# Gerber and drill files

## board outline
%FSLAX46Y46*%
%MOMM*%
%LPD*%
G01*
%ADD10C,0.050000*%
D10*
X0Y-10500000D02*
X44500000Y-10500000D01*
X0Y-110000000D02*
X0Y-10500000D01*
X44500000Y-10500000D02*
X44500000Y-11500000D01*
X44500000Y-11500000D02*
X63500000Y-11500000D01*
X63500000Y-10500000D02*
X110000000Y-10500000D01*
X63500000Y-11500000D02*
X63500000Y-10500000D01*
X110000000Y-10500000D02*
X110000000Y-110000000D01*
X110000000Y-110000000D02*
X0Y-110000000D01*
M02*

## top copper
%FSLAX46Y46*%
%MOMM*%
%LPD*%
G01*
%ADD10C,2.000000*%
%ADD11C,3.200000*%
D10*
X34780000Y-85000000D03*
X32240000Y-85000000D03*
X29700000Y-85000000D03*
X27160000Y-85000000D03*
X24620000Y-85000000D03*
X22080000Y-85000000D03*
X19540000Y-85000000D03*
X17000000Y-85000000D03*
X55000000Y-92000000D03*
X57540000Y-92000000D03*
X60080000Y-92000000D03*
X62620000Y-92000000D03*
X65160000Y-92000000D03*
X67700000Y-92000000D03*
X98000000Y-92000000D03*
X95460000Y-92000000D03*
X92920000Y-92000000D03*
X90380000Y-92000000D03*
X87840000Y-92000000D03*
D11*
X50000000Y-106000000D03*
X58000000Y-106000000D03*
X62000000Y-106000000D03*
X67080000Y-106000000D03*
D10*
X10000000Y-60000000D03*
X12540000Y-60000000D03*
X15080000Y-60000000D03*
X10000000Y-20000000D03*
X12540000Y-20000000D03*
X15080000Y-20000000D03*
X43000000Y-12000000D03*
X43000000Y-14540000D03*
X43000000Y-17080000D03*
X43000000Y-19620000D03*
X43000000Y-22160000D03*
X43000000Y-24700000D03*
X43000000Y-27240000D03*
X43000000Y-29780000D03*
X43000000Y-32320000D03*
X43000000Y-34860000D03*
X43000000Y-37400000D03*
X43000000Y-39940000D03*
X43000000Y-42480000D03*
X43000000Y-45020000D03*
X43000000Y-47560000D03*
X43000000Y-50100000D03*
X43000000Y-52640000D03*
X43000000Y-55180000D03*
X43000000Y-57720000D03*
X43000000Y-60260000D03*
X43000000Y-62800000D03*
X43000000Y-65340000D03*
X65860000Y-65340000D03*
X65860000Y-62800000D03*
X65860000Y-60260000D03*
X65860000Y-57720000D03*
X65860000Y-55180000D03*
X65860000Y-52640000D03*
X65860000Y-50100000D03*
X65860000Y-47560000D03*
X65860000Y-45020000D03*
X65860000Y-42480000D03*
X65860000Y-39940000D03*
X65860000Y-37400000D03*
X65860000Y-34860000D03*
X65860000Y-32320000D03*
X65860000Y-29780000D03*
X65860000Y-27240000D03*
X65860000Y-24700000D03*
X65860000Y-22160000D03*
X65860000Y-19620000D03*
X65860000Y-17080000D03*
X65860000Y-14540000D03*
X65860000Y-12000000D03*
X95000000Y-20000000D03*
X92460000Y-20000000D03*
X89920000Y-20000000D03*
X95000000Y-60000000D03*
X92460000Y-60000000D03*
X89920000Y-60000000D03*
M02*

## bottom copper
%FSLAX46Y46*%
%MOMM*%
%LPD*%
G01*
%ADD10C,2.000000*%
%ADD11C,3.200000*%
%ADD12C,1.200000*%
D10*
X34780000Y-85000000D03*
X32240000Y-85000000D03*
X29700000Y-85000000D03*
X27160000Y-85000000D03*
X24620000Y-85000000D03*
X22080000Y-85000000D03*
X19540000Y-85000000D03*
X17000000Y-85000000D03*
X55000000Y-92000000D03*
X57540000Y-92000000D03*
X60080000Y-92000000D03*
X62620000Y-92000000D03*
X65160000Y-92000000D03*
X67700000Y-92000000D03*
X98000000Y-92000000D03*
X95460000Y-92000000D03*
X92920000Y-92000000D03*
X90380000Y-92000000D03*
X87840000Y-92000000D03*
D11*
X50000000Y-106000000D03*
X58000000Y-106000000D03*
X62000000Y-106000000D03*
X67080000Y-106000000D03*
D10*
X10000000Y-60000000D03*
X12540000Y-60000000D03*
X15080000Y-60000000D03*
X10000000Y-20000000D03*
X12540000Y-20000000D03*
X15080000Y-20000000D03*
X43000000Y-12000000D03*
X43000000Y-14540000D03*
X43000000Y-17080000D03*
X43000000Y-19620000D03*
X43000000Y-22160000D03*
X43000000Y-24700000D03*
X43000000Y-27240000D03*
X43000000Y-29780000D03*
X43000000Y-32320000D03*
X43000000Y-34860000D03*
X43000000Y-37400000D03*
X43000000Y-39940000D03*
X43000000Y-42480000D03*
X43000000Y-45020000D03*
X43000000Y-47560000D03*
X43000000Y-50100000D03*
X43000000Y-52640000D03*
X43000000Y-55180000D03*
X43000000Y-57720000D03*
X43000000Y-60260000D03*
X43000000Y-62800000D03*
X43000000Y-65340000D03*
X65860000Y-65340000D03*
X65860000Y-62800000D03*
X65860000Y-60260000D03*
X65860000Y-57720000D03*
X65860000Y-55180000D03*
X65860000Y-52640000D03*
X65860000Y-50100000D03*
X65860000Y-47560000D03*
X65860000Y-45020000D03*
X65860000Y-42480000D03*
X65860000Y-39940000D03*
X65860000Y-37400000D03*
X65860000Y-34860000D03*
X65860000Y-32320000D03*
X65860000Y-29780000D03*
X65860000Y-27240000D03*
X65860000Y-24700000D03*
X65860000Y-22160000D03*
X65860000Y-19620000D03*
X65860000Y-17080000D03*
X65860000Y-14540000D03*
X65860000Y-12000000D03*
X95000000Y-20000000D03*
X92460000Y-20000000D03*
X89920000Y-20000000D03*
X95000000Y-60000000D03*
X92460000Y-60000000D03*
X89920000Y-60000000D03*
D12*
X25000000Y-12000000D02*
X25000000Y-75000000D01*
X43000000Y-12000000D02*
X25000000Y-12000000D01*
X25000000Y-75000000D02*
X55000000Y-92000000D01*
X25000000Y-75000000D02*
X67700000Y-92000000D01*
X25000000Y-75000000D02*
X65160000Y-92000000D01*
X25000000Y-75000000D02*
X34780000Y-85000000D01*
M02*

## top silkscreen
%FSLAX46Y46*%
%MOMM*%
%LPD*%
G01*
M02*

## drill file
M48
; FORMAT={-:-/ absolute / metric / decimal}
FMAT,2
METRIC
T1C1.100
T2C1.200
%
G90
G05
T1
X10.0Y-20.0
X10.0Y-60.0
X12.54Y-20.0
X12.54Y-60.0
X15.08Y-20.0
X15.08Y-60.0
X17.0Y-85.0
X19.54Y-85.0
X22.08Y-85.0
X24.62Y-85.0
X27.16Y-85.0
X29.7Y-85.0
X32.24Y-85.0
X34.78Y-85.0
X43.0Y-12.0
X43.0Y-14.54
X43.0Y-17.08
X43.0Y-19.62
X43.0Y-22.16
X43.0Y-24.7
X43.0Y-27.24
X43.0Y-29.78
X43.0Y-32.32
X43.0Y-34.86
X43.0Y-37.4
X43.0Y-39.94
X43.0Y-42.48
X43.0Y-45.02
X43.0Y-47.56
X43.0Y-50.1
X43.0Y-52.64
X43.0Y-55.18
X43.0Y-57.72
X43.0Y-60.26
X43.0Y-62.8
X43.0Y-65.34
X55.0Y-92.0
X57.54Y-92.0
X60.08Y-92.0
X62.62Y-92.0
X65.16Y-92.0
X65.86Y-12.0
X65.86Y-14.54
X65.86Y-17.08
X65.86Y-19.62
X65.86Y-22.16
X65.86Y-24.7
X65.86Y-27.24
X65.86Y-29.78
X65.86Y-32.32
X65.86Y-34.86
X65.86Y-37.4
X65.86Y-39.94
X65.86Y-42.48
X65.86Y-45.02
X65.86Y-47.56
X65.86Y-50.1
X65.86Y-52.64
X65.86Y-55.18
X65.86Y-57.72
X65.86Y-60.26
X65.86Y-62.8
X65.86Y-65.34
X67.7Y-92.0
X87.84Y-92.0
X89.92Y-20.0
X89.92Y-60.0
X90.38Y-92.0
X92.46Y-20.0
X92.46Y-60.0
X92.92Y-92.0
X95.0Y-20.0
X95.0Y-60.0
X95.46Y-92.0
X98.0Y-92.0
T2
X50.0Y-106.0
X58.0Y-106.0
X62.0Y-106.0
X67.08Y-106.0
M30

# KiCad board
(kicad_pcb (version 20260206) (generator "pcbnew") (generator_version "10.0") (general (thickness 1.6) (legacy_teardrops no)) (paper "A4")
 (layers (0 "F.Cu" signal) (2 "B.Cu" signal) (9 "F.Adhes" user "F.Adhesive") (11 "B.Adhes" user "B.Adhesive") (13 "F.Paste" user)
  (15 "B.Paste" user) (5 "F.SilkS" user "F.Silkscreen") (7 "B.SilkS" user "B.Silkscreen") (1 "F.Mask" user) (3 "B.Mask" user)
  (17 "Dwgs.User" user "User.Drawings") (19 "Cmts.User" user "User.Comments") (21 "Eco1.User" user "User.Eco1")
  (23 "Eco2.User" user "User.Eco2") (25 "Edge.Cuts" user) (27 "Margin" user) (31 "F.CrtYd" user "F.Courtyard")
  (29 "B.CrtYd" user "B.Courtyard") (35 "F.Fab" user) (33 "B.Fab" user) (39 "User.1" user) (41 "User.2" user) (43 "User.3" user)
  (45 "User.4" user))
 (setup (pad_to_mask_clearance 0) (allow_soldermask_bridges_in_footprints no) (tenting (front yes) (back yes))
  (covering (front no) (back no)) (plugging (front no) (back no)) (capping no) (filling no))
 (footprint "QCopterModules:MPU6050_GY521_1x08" (layer "F.Cu") (at 34.78 85 -90)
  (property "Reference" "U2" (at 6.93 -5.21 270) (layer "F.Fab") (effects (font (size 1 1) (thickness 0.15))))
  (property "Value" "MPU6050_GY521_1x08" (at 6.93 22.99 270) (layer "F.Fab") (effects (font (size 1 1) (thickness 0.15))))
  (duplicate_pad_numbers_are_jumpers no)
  (pad "1" thru_hole circle (at 0 0 270) (size 2 2) (drill 1.1) (layers "*.Cu" "*.Mask") (remove_unused_layers no) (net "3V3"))
  (pad "2" thru_hole circle (at 0 2.54 270) (size 2 2) (drill 1.1) (layers "*.Cu" "*.Mask") (remove_unused_layers no) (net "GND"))
  (pad "3" thru_hole circle (at 0 5.08 270) (size 2 2) (drill 1.1) (layers "*.Cu" "*.Mask") (remove_unused_layers no) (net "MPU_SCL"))
  (pad "4" thru_hole circle (at 0 7.62 270) (size 2 2) (drill 1.1) (layers "*.Cu" "*.Mask") (remove_unused_layers no) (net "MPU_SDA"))
  (pad "5" thru_hole circle (at 0 10.16 270) (size 2 2) (drill 1.1) (layers "*.Cu" "*.Mask") (remove_unused_layers no)
   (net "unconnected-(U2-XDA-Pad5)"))
  (pad "6" thru_hole circle (at 0 12.7 270) (size 2 2) (drill 1.1) (layers "*.Cu" "*.Mask") (remove_unused_layers no)
   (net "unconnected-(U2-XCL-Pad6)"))
  (pad "7" thru_hole circle (at 0 15.24 270) (size 2 2) (drill 1.1) (layers "*.Cu" "*.Mask") (remove_unused_layers no) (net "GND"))
  (pad "8" thru_hole circle (at 0 17.78 270) (size 2 2) (drill 1.1) (layers "*.Cu" "*.Mask") (remove_unused_layers no) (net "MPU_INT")))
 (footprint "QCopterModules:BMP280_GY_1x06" (layer "F.Cu") (at 55 92 90)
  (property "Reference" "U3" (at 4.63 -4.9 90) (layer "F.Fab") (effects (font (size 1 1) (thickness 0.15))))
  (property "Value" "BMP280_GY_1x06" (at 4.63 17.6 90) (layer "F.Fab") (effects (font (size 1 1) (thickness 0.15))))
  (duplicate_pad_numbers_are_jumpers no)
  (pad "1" thru_hole circle (at 0 0 90) (size 2 2) (drill 1.1) (layers "*.Cu" "*.Mask") (remove_unused_layers no) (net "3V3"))
  (pad "2" thru_hole circle (at 0 2.54 90) (size 2 2) (drill 1.1) (layers "*.Cu" "*.Mask") (remove_unused_layers no) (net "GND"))
  (pad "3" thru_hole circle (at 0 5.08 90) (size 2 2) (drill 1.1) (layers "*.Cu" "*.Mask") (remove_unused_layers no) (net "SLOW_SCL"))
  (pad "4" thru_hole circle (at 0 7.62 90) (size 2 2) (drill 1.1) (layers "*.Cu" "*.Mask") (remove_unused_layers no) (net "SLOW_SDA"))
  (pad "5" thru_hole circle (at 0 10.16 90) (size 2 2) (drill 1.1) (layers "*.Cu" "*.Mask") (remove_unused_layers no) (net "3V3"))
  (pad "6" thru_hole circle (at 0 12.7 90) (size 2 2) (drill 1.1) (layers "*.Cu" "*.Mask") (remove_unused_layers no) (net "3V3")))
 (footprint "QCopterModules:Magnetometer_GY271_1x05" (layer "F.Cu") (at 98 92 -90)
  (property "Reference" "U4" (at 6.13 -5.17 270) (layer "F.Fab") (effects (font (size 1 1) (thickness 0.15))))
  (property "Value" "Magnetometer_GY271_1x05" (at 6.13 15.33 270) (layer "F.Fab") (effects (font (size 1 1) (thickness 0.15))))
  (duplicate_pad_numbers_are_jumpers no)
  (pad "1" thru_hole circle (at 0 0 270) (size 2 2) (drill 1.1) (layers "*.Cu" "*.Mask") (remove_unused_layers no) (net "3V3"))
  (pad "2" thru_hole circle (at 0 2.54 270) (size 2 2) (drill 1.1) (layers "*.Cu" "*.Mask") (remove_unused_layers no) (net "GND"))
  (pad "3" thru_hole circle (at 0 5.08 270) (size 2 2) (drill 1.1) (layers "*.Cu" "*.Mask") (remove_unused_layers no) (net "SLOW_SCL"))
  (pad "4" thru_hole circle (at 0 7.62 270) (size 2 2) (drill 1.1) (layers "*.Cu" "*.Mask") (remove_unused_layers no) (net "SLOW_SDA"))
  (pad "5" thru_hole circle (at 0 10.16 270) (size 2 2) (drill 1.1) (layers "*.Cu" "*.Mask") (remove_unused_layers no) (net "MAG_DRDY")))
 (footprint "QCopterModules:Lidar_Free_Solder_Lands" (layer "F.Cu") (at 50 106)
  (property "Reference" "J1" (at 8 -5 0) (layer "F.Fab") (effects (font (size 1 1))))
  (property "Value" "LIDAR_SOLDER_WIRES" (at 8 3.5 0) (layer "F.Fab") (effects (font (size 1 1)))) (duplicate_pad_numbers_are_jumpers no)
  (pad "1" thru_hole circle (at 0 0) (size 3.2 3.2) (drill 1.2) (layers "*.Cu" "*.Mask") (remove_unused_layers no) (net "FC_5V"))
  (pad "2" thru_hole circle (at 8 0) (size 3.2 3.2) (drill 1.2) (layers "*.Cu" "*.Mask") (remove_unused_layers no) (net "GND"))
  (pad "3" thru_hole circle (at 12 0) (size 3.2 3.2) (drill 1.2) (layers "*.Cu" "*.Mask") (remove_unused_layers no) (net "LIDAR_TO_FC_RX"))
  (pad "4" thru_hole circle (at 17.08 0) (size 3.2 3.2) (drill 1.2) (layers "*.Cu" "*.Mask") (remove_unused_layers no)
   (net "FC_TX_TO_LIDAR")))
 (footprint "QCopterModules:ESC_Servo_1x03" (layer "F.Cu") (at 10 60 90)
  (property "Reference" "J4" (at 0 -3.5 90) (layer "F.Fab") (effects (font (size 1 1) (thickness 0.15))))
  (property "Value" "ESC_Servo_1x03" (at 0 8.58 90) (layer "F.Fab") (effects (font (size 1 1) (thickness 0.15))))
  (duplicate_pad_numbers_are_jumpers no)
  (pad "1" thru_hole circle (at 0 0 90) (size 2 2) (drill 1.1) (layers "*.Cu" "*.Mask") (remove_unused_layers no) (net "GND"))
  (pad "2" thru_hole circle (at 0 2.54 90) (size 2 2) (drill 1.1) (layers "*.Cu" "*.Mask") (remove_unused_layers no) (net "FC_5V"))
  (pad "3" thru_hole circle (at 0 5.08 90) (size 2 2) (drill 1.1) (layers "*.Cu" "*.Mask") (remove_unused_layers no) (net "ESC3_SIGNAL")))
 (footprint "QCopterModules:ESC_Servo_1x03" (layer "F.Cu") (at 10 20 90)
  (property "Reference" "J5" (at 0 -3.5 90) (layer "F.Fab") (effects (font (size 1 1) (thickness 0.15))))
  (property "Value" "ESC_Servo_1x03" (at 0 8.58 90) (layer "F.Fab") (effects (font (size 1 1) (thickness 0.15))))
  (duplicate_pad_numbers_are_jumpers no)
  (pad "1" thru_hole circle (at 0 0 90) (size 2 2) (drill 1.1) (layers "*.Cu" "*.Mask") (remove_unused_layers no) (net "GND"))
  (pad "2" thru_hole circle (at 0 2.54 90) (size 2 2) (drill 1.1) (layers "*.Cu" "*.Mask") (remove_unused_layers no)
   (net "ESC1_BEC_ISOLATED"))
  (pad "3" thru_hole circle (at 0 5.08 90) (size 2 2) (drill 1.1) (layers "*.Cu" "*.Mask") (remove_unused_layers no) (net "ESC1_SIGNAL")))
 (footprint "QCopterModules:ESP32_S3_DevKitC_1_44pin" (layer "F.Cu") (at 43 12)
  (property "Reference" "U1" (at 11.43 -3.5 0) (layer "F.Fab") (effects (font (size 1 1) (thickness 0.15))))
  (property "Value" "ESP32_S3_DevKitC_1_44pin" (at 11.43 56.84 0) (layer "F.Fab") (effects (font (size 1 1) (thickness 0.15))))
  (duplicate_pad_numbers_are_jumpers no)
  (pad "1" thru_hole circle (at 0 0) (size 2 2) (drill 1.1) (layers "*.Cu" "*.Mask") (remove_unused_layers no) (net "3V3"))
  (pad "2" thru_hole circle (at 0 2.54) (size 2 2) (drill 1.1) (layers "*.Cu" "*.Mask") (remove_unused_layers no))
  (pad "3" thru_hole circle (at 0 5.08) (size 2 2) (drill 1.1) (layers "*.Cu" "*.Mask") (remove_unused_layers no)
   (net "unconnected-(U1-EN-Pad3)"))
  (pad "4" thru_hole circle (at 0 7.62) (size 2 2) (drill 1.1) (layers "*.Cu" "*.Mask") (remove_unused_layers no) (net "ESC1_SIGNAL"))
  (pad "5" thru_hole circle (at 0 10.16) (size 2 2) (drill 1.1) (layers "*.Cu" "*.Mask") (remove_unused_layers no)
   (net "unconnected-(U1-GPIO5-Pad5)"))
  (pad "6" thru_hole circle (at 0 12.7) (size 2 2) (drill 1.1) (layers "*.Cu" "*.Mask") (remove_unused_layers no)
   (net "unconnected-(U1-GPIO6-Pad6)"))
  (pad "7" thru_hole circle (at 0 15.24) (size 2 2) (drill 1.1) (layers "*.Cu" "*.Mask") (remove_unused_layers no)
   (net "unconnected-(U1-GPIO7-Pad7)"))
  (pad "8" thru_hole circle (at 0 17.78) (size 2 2) (drill 1.1) (layers "*.Cu" "*.Mask") (remove_unused_layers no) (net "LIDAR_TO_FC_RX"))
  (pad "9" thru_hole circle (at 0 20.32) (size 2 2) (drill 1.1) (layers "*.Cu" "*.Mask") (remove_unused_layers no) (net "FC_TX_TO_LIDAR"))
  (pad "10" thru_hole circle (at 0 22.86) (size 2 2) (drill 1.1) (layers "*.Cu" "*.Mask") (remove_unused_layers no)
   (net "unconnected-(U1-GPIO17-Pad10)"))
  (pad "11" thru_hole circle (at 0 25.4) (size 2 2) (drill 1.1) (layers "*.Cu" "*.Mask") (remove_unused_layers no) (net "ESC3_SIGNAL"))
  (pad "12" thru_hole circle (at 0 27.94) (size 2 2) (drill 1.1) (layers "*.Cu" "*.Mask") (remove_unused_layers no)
   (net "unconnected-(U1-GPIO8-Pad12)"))
  (pad "13" thru_hole circle (at 0 30.48) (size 2 2) (drill 1.1) (layers "*.Cu" "*.Mask") (remove_unused_layers no)
   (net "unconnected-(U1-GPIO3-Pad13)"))
  (pad "14" thru_hole circle (at 0 33.02) (size 2 2) (drill 1.1) (layers "*.Cu" "*.Mask") (remove_unused_layers no)
   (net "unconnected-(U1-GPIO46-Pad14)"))
  (pad "15" thru_hole circle (at 0 35.56) (size 2 2) (drill 1.1) (layers "*.Cu" "*.Mask") (remove_unused_layers no)
   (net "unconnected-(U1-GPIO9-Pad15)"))
  (pad "16" thru_hole circle (at 0 38.1) (size 2 2) (drill 1.1) (layers "*.Cu" "*.Mask") (remove_unused_layers no)
   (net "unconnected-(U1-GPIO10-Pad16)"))
  (pad "17" thru_hole circle (at 0 40.64) (size 2 2) (drill 1.1) (layers "*.Cu" "*.Mask") (remove_unused_layers no)
   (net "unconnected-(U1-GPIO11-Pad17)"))
  (pad "18" thru_hole circle (at 0 43.18) (size 2 2) (drill 1.1) (layers "*.Cu" "*.Mask") (remove_unused_layers no) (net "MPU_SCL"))
  (pad "19" thru_hole circle (at 0 45.72) (size 2 2) (drill 1.1) (layers "*.Cu" "*.Mask") (remove_unused_layers no) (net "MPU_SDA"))
  (pad "20" thru_hole circle (at 0 48.26) (size 2 2) (drill 1.1) (layers "*.Cu" "*.Mask") (remove_unused_layers no) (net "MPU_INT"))
  (pad "21" thru_hole circle (at 0 50.8) (size 2 2) (drill 1.1) (layers "*.Cu" "*.Mask") (remove_unused_layers no) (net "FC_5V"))
  (pad "22" thru_hole circle (at 0 53.34) (size 2 2) (drill 1.1) (layers "*.Cu" "*.Mask") (remove_unused_layers no) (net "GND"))
  (pad "23" thru_hole circle (at 22.86 53.34) (size 2 2) (drill 1.1) (layers "*.Cu" "*.Mask") (remove_unused_layers no) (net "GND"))
  (pad "24" thru_hole circle (at 22.86 50.8) (size 2 2) (drill 1.1) (layers "*.Cu" "*.Mask") (remove_unused_layers no) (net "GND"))
  (pad "25" thru_hole circle (at 22.86 48.26) (size 2 2) (drill 1.1) (layers "*.Cu" "*.Mask") (remove_unused_layers no)
   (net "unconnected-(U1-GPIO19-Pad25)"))
  (pad "26" thru_hole circle (at 22.86 45.72) (size 2 2) (drill 1.1) (layers "*.Cu" "*.Mask") (remove_unused_layers no)
   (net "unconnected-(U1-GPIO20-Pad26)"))
  (pad "27" thru_hole circle (at 22.86 43.18) (size 2 2) (drill 1.1) (layers "*.Cu" "*.Mask") (remove_unused_layers no) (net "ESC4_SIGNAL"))
  (pad "28" thru_hole circle (at 22.86 40.64) (size 2 2) (drill 1.1) (layers "*.Cu" "*.Mask") (remove_unused_layers no)
   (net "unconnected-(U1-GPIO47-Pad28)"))
  (pad "29" thru_hole circle (at 22.86 38.1) (size 2 2) (drill 1.1) (layers "*.Cu" "*.Mask") (remove_unused_layers no)
   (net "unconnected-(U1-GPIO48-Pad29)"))
  (pad "30" thru_hole circle (at 22.86 35.56) (size 2 2) (drill 1.1) (layers "*.Cu" "*.Mask") (remove_unused_layers no)
   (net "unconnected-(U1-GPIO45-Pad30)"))
  (pad "31" thru_hole circle (at 22.86 33.02) (size 2 2) (drill 1.1) (layers "*.Cu" "*.Mask") (remove_unused_layers no)
   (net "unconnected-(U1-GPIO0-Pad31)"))
  (pad "32" thru_hole circle (at 22.86 30.48) (size 2 2) (drill 1.1) (layers "*.Cu" "*.Mask") (remove_unused_layers no)
   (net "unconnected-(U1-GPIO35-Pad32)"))
  (pad "33" thru_hole circle (at 22.86 27.94) (size 2 2) (drill 1.1) (layers "*.Cu" "*.Mask") (remove_unused_layers no)
   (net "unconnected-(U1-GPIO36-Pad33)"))
  (pad "34" thru_hole circle (at 22.86 25.4) (size 2 2) (drill 1.1) (layers "*.Cu" "*.Mask") (remove_unused_layers no)
   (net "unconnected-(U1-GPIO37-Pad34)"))
  (pad "35" thru_hole circle (at 22.86 22.86) (size 2 2) (drill 1.1) (layers "*.Cu" "*.Mask") (remove_unused_layers no)
   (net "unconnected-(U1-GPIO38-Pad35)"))
  (pad "36" thru_hole circle (at 22.86 20.32) (size 2 2) (drill 1.1) (layers "*.Cu" "*.Mask") (remove_unused_layers no) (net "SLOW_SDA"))
  (pad "37" thru_hole circle (at 22.86 17.78) (size 2 2) (drill 1.1) (layers "*.Cu" "*.Mask") (remove_unused_layers no) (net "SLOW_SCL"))
  (pad "38" thru_hole circle (at 22.86 15.24) (size 2 2) (drill 1.1) (layers "*.Cu" "*.Mask") (remove_unused_layers no) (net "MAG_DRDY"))
  (pad "39" thru_hole circle (at 22.86 12.7) (size 2 2) (drill 1.1) (layers "*.Cu" "*.Mask") (remove_unused_layers no)
   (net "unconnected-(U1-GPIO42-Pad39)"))
  (pad "40" thru_hole circle (at 22.86 10.16) (size 2 2) (drill 1.1) (layers "*.Cu" "*.Mask") (remove_unused_layers no) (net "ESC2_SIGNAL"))
  (pad "41" thru_hole circle (at 22.86 7.62) (size 2 2) (drill 1.1) (layers "*.Cu" "*.Mask") (remove_unused_layers no)
   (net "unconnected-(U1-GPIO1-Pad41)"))
  (pad "42" thru_hole circle (at 22.86 5.08) (size 2 2) (drill 1.1) (layers "*.Cu" "*.Mask") (remove_unused_layers no)
   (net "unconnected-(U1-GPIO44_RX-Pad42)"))
  (pad "43" thru_hole circle (at 22.86 2.54) (size 2 2) (drill 1.1) (layers "*.Cu" "*.Mask") (remove_unused_layers no)
   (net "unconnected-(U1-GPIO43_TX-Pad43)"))
  (pad "44" thru_hole circle (at 22.86 0) (size 2 2) (drill 1.1) (layers "*.Cu" "*.Mask") (remove_unused_layers no) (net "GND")))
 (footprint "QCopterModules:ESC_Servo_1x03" (layer "F.Cu") (at 95 20 -90)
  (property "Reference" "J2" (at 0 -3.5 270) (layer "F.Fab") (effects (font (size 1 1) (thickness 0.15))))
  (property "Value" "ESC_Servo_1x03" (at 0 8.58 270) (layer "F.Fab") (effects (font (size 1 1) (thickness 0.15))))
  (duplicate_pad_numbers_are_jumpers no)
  (pad "1" thru_hole circle (at 0 0 270) (size 2 2) (drill 1.1) (layers "*.Cu" "*.Mask") (remove_unused_layers no) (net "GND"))
  (pad "2" thru_hole circle (at 0 2.54 270) (size 2 2) (drill 1.1) (layers "*.Cu" "*.Mask") (remove_unused_layers no)
   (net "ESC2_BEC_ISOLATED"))
  (pad "3" thru_hole circle (at 0 5.08 270) (size 2 2) (drill 1.1) (layers "*.Cu" "*.Mask") (remove_unused_layers no) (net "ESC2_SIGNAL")))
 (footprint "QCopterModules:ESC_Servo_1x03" (layer "F.Cu") (at 95 60 -90)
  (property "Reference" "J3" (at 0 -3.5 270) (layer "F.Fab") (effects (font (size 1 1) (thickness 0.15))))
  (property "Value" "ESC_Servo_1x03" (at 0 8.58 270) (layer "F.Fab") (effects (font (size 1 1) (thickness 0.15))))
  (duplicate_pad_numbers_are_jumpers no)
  (pad "1" thru_hole circle (at 0 0 270) (size 2 2) (drill 1.1) (layers "*.Cu" "*.Mask") (remove_unused_layers no) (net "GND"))
  (pad "2" thru_hole circle (at 0 2.54 270) (size 2 2) (drill 1.1) (layers "*.Cu" "*.Mask") (remove_unused_layers no)
   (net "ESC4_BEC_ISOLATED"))
  (pad "3" thru_hole circle (at 0 5.08 270) (size 2 2) (drill 1.1) (layers "*.Cu" "*.Mask") (remove_unused_layers no) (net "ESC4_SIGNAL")))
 (gr_line (start 0 10.5) (end 44.5 10.5) (stroke (width 0.05) (type default)) (layer "Edge.Cuts"))
 (gr_line (start 0 110) (end 0 10.5) (stroke (width 0.05) (type default)) (layer "Edge.Cuts"))
 (gr_line (start 44.5 10.5) (end 44.5 11.5) (stroke (width 0.05) (type default)) (layer "Edge.Cuts"))
 (gr_line (start 44.5 11.5) (end 63.5 11.5) (stroke (width 0.05) (type default)) (layer "Edge.Cuts"))
 (gr_line (start 63.5 10.5) (end 110 10.5) (stroke (width 0.05) (type default)) (layer "Edge.Cuts"))
 (gr_line (start 63.5 11.5) (end 63.5 10.5) (stroke (width 0.05) (type default)) (layer "Edge.Cuts"))
 (gr_line (start 110 10.5) (end 110 110) (stroke (width 0.05) (type default)) (layer "Edge.Cuts"))
 (gr_line (start 110 110) (end 0 110) (stroke (width 0.05) (type default)) (layer "Edge.Cuts"))
 (segment (start 25 12) (end 25 75) (width 1.2) (layer "B.Cu") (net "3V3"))
 (segment (start 43 12) (end 25 12) (width 1.2) (layer "B.Cu") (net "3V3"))
 (segment (start 25 75) (end 55 92) (width 1.2) (layer "B.Cu") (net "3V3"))
 (segment (start 25 75) (end 67.7 92) (width 1.2) (layer "B.Cu") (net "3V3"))
 (segment (start 25 75) (end 65.16 92) (width 1.2) (layer "B.Cu") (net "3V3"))
 (segment (start 25 75) (end 34.78 85) (width 1.2) (layer "B.Cu") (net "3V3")))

